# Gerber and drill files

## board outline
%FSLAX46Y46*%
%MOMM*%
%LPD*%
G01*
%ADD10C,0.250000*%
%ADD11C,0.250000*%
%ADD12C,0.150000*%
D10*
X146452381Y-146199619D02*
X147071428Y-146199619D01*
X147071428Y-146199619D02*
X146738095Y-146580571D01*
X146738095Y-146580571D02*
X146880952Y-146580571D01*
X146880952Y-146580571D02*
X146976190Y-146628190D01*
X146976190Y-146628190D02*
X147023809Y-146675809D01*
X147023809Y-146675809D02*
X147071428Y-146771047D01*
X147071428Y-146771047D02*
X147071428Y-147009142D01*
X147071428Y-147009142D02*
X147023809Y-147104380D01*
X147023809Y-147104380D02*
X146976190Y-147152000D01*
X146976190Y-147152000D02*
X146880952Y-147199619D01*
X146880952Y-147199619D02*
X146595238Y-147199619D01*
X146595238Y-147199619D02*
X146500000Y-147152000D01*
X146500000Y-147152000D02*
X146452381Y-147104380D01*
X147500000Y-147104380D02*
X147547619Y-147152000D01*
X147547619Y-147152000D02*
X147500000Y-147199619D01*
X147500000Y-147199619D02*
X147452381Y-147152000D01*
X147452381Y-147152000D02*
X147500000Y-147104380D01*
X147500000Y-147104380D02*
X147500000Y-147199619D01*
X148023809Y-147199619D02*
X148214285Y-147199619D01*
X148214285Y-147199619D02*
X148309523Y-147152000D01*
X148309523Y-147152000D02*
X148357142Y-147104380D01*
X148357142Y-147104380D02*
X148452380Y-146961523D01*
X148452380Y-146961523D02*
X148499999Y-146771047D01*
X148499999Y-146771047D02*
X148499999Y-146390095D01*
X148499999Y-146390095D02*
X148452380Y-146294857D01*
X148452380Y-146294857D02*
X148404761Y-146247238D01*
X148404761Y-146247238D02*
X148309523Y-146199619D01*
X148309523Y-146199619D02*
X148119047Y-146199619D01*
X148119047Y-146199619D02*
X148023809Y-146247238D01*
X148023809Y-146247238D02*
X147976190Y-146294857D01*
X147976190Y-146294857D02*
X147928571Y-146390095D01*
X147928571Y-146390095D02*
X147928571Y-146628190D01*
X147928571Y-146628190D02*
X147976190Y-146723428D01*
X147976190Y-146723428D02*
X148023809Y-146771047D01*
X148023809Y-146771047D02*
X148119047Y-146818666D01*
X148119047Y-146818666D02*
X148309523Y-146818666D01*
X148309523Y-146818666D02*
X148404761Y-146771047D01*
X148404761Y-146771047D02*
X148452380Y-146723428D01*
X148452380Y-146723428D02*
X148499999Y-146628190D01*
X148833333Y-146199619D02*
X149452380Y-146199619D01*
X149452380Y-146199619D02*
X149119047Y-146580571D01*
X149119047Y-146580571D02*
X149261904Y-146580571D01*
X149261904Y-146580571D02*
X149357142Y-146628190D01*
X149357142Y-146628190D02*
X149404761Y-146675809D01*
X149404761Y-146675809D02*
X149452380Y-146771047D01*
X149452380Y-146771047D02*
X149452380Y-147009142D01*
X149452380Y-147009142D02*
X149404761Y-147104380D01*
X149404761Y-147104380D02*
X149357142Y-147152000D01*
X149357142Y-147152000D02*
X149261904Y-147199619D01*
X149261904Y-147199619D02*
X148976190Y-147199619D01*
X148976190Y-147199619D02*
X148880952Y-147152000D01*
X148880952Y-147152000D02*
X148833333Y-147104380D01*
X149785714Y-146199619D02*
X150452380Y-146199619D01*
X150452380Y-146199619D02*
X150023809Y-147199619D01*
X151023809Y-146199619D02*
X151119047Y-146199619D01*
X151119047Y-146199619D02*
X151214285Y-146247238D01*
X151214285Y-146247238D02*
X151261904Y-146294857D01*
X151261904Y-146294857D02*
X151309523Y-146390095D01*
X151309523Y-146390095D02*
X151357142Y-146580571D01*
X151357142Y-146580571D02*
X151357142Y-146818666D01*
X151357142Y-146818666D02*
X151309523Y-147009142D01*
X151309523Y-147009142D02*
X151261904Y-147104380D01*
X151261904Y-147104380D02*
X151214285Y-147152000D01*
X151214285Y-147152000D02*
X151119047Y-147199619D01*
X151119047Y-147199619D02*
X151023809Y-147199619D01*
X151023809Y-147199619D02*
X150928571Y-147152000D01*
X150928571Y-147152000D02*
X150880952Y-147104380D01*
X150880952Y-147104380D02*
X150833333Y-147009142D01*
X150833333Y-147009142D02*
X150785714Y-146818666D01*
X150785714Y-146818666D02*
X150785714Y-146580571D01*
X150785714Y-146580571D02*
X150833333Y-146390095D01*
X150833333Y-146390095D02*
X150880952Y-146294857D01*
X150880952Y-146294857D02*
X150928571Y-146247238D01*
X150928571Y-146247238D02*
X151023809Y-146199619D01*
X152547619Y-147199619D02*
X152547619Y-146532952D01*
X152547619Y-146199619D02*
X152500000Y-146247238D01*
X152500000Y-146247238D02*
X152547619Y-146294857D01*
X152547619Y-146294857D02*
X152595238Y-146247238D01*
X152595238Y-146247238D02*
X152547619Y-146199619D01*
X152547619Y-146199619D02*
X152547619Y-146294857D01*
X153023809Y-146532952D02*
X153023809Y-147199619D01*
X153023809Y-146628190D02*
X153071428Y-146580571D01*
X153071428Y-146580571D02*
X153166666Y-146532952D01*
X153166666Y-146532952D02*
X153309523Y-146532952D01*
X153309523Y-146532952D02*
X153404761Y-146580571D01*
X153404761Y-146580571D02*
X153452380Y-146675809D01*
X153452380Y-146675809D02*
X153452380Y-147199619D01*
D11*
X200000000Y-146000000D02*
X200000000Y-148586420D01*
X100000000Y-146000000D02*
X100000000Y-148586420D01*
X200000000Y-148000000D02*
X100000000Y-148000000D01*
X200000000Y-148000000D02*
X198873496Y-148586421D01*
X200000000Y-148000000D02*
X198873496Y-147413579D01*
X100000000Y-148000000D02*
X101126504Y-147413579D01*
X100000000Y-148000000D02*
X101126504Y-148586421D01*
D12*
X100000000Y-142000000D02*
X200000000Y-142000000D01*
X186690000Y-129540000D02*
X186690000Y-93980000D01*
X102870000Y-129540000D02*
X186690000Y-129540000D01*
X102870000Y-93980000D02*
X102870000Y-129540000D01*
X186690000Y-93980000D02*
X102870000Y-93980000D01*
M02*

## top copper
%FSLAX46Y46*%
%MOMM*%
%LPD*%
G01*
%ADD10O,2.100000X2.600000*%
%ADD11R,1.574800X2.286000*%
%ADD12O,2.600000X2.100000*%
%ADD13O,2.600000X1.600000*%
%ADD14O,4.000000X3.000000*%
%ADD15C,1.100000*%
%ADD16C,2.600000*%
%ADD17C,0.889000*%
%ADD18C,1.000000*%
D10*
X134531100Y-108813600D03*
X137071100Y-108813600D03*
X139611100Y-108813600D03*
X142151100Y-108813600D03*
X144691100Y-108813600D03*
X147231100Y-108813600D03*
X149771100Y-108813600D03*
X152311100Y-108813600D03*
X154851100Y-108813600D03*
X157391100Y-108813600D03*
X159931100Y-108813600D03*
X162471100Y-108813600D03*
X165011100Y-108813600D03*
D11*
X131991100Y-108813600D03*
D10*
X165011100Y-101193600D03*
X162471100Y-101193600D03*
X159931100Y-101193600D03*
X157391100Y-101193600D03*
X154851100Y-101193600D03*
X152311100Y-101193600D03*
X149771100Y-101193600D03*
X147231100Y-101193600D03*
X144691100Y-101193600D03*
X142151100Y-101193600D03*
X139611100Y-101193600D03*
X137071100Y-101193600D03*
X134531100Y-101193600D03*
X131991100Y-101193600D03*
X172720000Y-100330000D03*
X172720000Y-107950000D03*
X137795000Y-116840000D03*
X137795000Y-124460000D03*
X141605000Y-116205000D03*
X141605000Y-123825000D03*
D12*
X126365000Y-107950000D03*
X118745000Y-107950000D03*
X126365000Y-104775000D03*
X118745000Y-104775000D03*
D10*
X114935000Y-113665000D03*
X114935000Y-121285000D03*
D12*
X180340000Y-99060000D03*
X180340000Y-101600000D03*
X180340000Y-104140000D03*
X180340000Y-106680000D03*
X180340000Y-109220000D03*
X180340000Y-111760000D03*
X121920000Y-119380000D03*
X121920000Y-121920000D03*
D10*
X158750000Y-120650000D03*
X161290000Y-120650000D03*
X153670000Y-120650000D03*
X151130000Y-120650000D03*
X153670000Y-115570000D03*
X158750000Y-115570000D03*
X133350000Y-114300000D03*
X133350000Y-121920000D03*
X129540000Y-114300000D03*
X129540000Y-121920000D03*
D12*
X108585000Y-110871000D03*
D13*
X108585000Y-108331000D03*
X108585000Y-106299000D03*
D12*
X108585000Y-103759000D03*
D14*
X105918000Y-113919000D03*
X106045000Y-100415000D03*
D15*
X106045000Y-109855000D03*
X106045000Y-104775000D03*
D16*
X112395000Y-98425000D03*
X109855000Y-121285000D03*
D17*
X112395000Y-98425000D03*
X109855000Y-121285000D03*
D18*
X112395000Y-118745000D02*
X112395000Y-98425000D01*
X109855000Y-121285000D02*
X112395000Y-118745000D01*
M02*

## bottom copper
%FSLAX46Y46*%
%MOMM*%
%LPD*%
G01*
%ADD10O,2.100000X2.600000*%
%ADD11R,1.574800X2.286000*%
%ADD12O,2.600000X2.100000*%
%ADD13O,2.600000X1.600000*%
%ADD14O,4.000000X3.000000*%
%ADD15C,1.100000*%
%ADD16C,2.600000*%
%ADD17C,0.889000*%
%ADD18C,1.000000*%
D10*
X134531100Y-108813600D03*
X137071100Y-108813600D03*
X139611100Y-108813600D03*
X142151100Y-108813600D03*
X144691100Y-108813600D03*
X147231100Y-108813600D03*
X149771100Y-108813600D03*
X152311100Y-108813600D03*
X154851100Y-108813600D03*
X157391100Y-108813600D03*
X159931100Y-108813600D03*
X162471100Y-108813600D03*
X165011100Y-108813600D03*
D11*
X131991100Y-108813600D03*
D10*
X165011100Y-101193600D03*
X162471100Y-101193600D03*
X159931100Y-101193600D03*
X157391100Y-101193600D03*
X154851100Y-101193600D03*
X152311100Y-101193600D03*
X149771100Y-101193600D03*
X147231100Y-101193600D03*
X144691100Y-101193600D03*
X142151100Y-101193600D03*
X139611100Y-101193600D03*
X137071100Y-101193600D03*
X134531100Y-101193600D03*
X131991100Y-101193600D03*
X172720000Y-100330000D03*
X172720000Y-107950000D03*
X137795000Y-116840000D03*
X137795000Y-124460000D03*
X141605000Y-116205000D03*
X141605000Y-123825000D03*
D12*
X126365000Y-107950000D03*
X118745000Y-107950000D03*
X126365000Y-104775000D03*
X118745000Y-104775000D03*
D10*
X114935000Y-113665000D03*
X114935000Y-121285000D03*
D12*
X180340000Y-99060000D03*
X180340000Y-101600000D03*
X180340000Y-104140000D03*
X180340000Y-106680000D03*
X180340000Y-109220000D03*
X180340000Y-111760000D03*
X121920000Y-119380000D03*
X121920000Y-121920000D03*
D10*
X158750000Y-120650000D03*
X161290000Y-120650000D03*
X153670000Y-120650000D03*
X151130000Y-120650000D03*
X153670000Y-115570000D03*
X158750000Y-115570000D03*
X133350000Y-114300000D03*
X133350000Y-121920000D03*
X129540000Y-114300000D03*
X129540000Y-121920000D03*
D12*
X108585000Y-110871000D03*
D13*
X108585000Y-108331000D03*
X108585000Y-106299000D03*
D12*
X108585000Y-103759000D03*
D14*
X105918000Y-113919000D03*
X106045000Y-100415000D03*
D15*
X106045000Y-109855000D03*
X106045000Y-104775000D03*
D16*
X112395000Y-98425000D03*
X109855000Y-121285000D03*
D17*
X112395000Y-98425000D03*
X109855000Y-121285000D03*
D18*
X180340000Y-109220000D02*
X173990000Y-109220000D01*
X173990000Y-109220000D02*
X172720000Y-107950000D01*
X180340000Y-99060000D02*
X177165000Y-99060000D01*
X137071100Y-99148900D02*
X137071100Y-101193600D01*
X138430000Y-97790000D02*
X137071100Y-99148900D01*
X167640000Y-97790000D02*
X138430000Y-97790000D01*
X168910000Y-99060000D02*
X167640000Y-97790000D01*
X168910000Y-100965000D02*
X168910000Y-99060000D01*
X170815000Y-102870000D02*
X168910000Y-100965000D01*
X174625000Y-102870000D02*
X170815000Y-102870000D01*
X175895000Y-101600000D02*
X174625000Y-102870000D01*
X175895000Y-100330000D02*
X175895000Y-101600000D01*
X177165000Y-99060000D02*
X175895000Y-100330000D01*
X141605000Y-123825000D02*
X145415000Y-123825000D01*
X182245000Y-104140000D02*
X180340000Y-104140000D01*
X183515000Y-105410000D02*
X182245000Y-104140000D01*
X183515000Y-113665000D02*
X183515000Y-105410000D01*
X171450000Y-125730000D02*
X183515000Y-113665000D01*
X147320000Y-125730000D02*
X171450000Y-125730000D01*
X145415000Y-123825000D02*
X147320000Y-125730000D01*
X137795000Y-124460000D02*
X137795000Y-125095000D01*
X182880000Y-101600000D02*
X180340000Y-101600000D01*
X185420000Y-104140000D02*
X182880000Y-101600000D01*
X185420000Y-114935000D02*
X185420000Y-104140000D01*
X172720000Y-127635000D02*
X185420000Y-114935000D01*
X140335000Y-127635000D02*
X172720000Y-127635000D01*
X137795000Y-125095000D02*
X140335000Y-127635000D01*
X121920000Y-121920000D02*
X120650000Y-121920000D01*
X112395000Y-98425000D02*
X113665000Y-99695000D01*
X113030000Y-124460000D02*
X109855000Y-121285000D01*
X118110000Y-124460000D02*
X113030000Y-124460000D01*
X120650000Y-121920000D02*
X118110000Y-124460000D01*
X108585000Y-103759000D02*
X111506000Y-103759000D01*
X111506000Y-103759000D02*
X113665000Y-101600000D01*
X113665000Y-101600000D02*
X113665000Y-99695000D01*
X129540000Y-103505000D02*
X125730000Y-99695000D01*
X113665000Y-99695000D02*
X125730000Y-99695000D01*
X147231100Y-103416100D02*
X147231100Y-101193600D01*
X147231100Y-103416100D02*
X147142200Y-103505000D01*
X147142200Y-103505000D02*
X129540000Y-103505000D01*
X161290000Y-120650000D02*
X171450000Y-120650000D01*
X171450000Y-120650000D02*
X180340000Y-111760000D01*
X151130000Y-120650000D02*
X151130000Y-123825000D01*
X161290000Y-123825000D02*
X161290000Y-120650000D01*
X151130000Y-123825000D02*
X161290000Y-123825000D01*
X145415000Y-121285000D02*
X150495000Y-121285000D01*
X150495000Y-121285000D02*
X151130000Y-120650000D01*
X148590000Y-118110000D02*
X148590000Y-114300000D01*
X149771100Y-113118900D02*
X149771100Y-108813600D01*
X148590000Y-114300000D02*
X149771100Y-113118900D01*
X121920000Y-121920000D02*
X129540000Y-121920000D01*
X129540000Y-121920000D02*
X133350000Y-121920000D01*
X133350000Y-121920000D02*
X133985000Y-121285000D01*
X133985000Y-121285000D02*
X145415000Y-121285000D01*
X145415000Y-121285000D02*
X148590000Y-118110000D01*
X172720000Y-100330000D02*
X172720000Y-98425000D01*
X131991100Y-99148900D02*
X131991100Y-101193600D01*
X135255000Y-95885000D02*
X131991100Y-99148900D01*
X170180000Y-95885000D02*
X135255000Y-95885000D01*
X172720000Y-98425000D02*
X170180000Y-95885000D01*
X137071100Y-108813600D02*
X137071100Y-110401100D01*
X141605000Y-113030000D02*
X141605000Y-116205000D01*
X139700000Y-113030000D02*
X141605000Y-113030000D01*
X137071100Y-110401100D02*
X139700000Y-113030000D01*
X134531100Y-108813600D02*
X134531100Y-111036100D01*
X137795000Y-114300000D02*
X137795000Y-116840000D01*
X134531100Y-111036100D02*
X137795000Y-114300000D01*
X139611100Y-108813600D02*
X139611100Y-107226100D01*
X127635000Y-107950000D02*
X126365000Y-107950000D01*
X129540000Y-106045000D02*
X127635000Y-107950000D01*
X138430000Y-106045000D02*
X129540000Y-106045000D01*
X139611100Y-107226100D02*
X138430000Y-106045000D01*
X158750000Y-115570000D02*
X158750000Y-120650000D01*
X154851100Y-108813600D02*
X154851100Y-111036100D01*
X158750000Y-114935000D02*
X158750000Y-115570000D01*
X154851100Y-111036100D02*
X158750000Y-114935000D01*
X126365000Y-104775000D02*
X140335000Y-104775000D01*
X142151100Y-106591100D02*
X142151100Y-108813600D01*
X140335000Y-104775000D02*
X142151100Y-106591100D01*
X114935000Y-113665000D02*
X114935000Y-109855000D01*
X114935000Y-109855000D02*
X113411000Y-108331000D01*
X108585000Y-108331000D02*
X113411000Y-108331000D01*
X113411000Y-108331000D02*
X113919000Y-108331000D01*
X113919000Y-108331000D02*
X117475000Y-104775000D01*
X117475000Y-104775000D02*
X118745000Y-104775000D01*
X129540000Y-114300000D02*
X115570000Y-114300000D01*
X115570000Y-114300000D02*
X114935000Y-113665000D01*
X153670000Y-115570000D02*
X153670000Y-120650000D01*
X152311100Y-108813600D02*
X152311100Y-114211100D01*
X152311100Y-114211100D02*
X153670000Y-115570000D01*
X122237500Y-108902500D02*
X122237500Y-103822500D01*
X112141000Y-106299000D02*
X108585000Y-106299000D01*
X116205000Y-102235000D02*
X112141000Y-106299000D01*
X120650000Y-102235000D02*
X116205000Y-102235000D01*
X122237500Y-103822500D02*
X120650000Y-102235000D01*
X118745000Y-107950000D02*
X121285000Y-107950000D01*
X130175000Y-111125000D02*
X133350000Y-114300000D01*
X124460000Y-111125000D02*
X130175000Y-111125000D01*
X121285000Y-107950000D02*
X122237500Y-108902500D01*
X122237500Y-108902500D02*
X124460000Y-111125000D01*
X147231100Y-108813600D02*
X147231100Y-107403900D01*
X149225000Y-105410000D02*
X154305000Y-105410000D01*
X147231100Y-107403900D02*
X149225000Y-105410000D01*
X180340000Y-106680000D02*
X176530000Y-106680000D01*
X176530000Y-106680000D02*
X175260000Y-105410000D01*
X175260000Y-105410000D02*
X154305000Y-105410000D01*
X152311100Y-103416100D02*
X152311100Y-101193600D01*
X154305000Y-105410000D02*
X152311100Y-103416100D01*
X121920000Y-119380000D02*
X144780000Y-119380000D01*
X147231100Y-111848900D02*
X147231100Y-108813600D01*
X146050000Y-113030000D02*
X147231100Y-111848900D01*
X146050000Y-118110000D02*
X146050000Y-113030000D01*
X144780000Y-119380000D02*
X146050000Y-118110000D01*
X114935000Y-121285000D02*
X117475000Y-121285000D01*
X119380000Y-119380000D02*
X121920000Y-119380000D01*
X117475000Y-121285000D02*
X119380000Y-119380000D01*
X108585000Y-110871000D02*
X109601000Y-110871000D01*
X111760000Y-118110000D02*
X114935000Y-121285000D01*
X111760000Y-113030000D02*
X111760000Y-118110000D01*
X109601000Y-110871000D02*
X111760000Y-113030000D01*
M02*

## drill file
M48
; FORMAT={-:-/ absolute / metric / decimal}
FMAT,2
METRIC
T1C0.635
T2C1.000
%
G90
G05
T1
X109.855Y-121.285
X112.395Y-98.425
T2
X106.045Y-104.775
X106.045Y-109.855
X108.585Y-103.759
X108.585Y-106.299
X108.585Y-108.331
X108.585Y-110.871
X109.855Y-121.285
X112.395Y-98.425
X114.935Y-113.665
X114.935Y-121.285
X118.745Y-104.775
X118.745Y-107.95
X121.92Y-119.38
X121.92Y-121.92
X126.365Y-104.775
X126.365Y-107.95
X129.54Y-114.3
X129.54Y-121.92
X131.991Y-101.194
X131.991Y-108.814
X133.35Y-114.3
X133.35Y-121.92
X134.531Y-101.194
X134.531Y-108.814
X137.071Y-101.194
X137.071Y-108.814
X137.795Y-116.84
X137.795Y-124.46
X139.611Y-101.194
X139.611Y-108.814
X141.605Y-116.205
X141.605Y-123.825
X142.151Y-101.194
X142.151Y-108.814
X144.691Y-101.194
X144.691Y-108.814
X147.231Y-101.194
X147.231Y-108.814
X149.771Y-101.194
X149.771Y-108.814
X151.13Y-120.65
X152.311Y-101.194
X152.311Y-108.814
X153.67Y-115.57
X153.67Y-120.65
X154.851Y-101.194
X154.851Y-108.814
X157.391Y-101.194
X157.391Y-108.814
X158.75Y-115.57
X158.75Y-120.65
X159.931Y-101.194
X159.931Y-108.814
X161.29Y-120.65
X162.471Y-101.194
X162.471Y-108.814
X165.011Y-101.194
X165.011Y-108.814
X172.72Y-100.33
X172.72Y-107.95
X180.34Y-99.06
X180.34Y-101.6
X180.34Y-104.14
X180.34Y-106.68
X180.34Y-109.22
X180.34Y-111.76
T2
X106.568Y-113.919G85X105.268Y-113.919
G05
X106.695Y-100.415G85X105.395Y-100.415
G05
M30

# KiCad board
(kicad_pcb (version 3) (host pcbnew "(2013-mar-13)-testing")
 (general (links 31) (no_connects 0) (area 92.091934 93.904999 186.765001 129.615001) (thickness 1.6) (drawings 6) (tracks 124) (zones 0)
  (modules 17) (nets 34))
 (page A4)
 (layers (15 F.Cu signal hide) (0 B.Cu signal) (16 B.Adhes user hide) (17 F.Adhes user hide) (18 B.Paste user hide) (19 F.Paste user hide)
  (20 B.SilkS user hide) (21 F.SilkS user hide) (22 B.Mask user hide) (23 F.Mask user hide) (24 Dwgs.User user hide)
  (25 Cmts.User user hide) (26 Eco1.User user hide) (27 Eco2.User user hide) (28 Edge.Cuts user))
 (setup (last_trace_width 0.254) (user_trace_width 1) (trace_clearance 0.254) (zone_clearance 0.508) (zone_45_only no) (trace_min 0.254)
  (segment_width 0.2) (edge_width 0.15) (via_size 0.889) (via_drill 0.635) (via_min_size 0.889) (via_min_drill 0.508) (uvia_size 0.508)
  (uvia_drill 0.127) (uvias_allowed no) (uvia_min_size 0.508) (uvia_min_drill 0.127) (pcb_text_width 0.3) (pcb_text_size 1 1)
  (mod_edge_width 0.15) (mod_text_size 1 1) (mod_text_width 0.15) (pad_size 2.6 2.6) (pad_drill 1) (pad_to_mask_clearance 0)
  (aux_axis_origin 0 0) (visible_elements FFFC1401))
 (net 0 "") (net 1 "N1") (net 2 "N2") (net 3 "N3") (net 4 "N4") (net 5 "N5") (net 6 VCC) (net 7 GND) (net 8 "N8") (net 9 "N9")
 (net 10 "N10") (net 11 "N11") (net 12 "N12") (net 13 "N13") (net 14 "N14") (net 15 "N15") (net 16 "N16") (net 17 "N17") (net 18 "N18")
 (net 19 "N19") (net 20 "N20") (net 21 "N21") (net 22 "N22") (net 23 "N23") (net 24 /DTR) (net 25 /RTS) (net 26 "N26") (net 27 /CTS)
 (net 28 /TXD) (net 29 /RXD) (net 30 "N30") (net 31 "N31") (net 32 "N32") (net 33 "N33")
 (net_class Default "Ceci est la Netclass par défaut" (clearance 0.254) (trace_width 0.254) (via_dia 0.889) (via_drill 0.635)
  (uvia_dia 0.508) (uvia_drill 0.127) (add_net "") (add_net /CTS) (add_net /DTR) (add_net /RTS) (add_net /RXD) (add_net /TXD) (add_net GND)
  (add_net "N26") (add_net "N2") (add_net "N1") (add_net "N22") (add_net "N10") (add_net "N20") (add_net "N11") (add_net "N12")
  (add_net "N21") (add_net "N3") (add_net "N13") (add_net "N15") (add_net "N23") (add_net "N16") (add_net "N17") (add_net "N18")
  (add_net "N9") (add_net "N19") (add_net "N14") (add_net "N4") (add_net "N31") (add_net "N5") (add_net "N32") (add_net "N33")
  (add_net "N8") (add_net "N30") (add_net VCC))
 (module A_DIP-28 (layer F.Cu) (at 148.5011 105.0036)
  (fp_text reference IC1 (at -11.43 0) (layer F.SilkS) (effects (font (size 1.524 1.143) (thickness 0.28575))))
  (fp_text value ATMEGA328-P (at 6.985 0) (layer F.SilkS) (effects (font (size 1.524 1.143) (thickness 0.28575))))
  (pad 2 thru_hole oval (at -13.97 3.81) (size 2.1 2.6) (drill 1) (layers *.Cu *.Mask F.SilkS) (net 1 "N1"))
  (pad 3 thru_hole oval (at -11.43 3.81) (size 2.1 2.6) (drill 1) (layers *.Cu *.Mask F.SilkS) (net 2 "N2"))
  (pad 4 thru_hole oval (at -8.89 3.81) (size 2.1 2.6) (drill 1) (layers *.Cu *.Mask F.SilkS) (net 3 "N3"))
  (pad 5 thru_hole oval (at -6.35 3.81) (size 2.1 2.6) (drill 1) (layers *.Cu *.Mask F.SilkS) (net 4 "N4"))
  (pad 6 thru_hole oval (at -3.81 3.81) (size 2.1 2.6) (drill 1) (layers *.Cu *.Mask F.SilkS) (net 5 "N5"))
  (pad 7 thru_hole oval (at -1.27 3.81) (size 2.1 2.6) (drill 1) (layers *.Cu *.Mask F.SilkS) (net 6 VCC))
  (pad 8 thru_hole oval (at 1.27 3.81) (size 2.1 2.6) (drill 1) (layers *.Cu *.Mask F.SilkS) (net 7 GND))
  (pad 9 thru_hole oval (at 3.81 3.81) (size 2.1 2.6) (drill 1) (layers *.Cu *.Mask F.SilkS) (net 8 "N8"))
  (pad 10 thru_hole oval (at 6.35 3.81) (size 2.1 2.6) (drill 1) (layers *.Cu *.Mask F.SilkS) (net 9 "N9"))
  (pad 11 thru_hole oval (at 8.89 3.81) (size 2.1 2.6) (drill 1) (layers *.Cu *.Mask F.SilkS) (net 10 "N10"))
  (pad 12 thru_hole oval (at 11.43 3.81) (size 2.1 2.6) (drill 1) (layers *.Cu *.Mask F.SilkS) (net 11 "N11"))
  (pad 13 thru_hole oval (at 13.97 3.81) (size 2.1 2.6) (drill 1) (layers *.Cu *.Mask F.SilkS) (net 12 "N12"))
  (pad 14 thru_hole oval (at 16.51 3.81) (size 2.1 2.6) (drill 1) (layers *.Cu *.Mask F.SilkS) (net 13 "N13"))
  (pad 1 thru_hole rect (at -16.51 3.81) (size 1.5748 2.286) (drill 1) (layers *.Cu *.Mask F.SilkS) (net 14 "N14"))
  (pad 15 thru_hole oval (at 16.51 -3.81) (size 2.1 2.6) (drill 1) (layers *.Cu *.Mask F.SilkS) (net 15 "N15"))
  (pad 16 thru_hole oval (at 13.97 -3.81) (size 2.1 2.6) (drill 1) (layers *.Cu *.Mask F.SilkS) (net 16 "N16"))
  (pad 17 thru_hole oval (at 11.43 -3.81) (size 2.1 2.6) (drill 1) (layers *.Cu *.Mask F.SilkS) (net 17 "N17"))
  (pad 18 thru_hole oval (at 8.89 -3.81) (size 2.1 2.6) (drill 1) (layers *.Cu *.Mask F.SilkS) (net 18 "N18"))
  (pad 19 thru_hole oval (at 6.35 -3.81) (size 2.1 2.6) (drill 1) (layers *.Cu *.Mask F.SilkS) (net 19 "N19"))
  (pad 20 thru_hole oval (at 3.81 -3.81) (size 2.1 2.6) (drill 1) (layers *.Cu *.Mask F.SilkS) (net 6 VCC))
  (pad 21 thru_hole oval (at 1.27 -3.81) (size 2.1 2.6) (drill 1) (layers *.Cu *.Mask F.SilkS) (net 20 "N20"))
  (pad 22 thru_hole oval (at -1.27 -3.81) (size 2.1 2.6) (drill 1) (layers *.Cu *.Mask F.SilkS) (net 7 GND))
  (pad 23 thru_hole oval (at -3.81 -3.81) (size 2.1 2.6) (drill 1) (layers *.Cu *.Mask F.SilkS) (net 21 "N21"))
  (pad 24 thru_hole oval (at -6.35 -3.81) (size 2.1 2.6) (drill 1) (layers *.Cu *.Mask F.SilkS) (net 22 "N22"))
  (pad 25 thru_hole oval (at -8.89 -3.81) (size 2.1 2.6) (drill 1) (layers *.Cu *.Mask F.SilkS) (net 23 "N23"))
  (pad 26 thru_hole oval (at -11.43 -3.81) (size 2.1 2.6) (drill 1) (layers *.Cu *.Mask F.SilkS) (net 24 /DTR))
  (pad 27 thru_hole oval (at -13.97 -3.81) (size 2.1 2.6) (drill 1) (layers *.Cu *.Mask F.SilkS) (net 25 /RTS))
  (pad 28 thru_hole oval (at -16.51 -3.81) (size 2.1 2.6) (drill 1) (layers *.Cu *.Mask F.SilkS) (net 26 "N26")))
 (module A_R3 (layer F.Cu) (at 172.72 104.14 270) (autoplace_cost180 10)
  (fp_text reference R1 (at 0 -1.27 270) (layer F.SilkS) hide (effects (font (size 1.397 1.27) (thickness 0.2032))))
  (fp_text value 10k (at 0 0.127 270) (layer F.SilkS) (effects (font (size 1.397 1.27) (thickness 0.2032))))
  (pad 1 thru_hole oval (at -3.81 0 270) (size 2.6 2.1) (drill 1) (layers *.Cu *.Mask F.SilkS) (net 26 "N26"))
  (pad 2 thru_hole oval (at 3.81 0 270) (size 2.6 2.1) (drill 1) (layers *.Cu *.Mask F.SilkS) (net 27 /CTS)))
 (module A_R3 (layer F.Cu) (at 137.795 120.65 270) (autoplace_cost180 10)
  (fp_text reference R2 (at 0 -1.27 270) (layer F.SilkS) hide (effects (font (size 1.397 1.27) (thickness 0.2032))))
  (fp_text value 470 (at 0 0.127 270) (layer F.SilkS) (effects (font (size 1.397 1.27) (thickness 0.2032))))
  (pad 1 thru_hole oval (at -3.81 0 270) (size 2.6 2.1) (drill 1) (layers *.Cu *.Mask F.SilkS) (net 1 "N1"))
  (pad 2 thru_hole oval (at 3.81 0 270) (size 2.6 2.1) (drill 1) (layers *.Cu *.Mask F.SilkS) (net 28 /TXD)))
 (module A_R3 (layer F.Cu) (at 141.605 120.015 270) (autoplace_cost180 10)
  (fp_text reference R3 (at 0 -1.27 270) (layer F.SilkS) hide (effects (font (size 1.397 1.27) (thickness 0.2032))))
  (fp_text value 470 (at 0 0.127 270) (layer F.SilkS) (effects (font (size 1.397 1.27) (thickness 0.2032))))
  (pad 1 thru_hole oval (at -3.81 0 270) (size 2.6 2.1) (drill 1) (layers *.Cu *.Mask F.SilkS) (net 2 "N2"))
  (pad 2 thru_hole oval (at 3.81 0 270) (size 2.6 2.1) (drill 1) (layers *.Cu *.Mask F.SilkS) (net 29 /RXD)))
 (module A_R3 (layer F.Cu) (at 122.555 107.95 180) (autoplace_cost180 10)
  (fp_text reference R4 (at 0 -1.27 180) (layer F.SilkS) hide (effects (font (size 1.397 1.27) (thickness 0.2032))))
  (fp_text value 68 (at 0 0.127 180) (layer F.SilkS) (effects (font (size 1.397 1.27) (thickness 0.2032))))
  (pad 1 thru_hole oval (at -3.81 0 180) (size 2.6 2.1) (drill 1) (layers *.Cu *.Mask F.SilkS) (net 3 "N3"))
  (pad 2 thru_hole oval (at 3.81 0 180) (size 2.6 2.1) (drill 1) (layers *.Cu *.Mask F.SilkS) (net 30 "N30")))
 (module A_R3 (layer F.Cu) (at 122.555 104.775 180) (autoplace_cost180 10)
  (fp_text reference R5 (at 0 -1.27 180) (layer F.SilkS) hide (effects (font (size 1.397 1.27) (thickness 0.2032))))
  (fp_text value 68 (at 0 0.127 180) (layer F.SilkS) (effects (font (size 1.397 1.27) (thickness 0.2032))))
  (pad 1 thru_hole oval (at -3.81 0 180) (size 2.6 2.1) (drill 1) (layers *.Cu *.Mask F.SilkS) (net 4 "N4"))
  (pad 2 thru_hole oval (at 3.81 0 180) (size 2.6 2.1) (drill 1) (layers *.Cu *.Mask F.SilkS) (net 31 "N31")))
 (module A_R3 (layer F.Cu) (at 114.935 117.475 270) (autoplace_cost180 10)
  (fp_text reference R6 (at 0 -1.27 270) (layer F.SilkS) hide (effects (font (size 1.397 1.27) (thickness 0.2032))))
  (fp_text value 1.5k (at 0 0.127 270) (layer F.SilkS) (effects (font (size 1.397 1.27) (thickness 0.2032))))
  (pad 1 thru_hole oval (at -3.81 0 270) (size 2.6 2.1) (drill 1) (layers *.Cu *.Mask F.SilkS) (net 31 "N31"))
  (pad 2 thru_hole oval (at 3.81 0 270) (size 2.6 2.1) (drill 1) (layers *.Cu *.Mask F.SilkS) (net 6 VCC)))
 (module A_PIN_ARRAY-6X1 (layer F.Cu) (at 180.34 105.41 270)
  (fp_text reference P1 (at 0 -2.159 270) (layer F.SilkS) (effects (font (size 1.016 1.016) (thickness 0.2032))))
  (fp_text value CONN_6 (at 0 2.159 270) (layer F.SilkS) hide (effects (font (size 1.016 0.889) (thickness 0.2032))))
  (pad 1 thru_hole oval (at -6.35 0 270) (size 2.1 2.6) (drill 1) (layers *.Cu *.Mask F.SilkS) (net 24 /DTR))
  (pad 2 thru_hole oval (at -3.81 0 270) (size 2.1 2.6) (drill 1) (layers *.Cu *.Mask F.SilkS) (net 28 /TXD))
  (pad 3 thru_hole oval (at -1.27 0 270) (size 2.1 2.6) (drill 1) (layers *.Cu *.Mask F.SilkS) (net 29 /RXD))
  (pad 4 thru_hole oval (at 1.27 0 270) (size 2.1 2.6) (drill 1) (layers *.Cu *.Mask F.SilkS) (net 6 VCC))
  (pad 5 thru_hole oval (at 3.81 0 270) (size 2.1 2.6) (drill 1) (layers *.Cu *.Mask F.SilkS) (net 27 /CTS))
  (pad 6 thru_hole oval (at 6.35 0 270) (size 2.1 2.6) (drill 1) (layers *.Cu *.Mask F.SilkS) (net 7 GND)))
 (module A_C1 (layer F.Cu) (at 121.92 120.65 270)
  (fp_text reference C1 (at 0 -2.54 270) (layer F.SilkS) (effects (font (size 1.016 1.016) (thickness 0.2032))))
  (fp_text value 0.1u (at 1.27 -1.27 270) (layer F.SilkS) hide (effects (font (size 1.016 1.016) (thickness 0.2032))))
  (pad 1 thru_hole oval (at -1.27 0 270) (size 2.1 2.6) (drill 1) (layers *.Cu *.Mask F.SilkS) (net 6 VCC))
  (pad 2 thru_hole oval (at 1.27 0 270) (size 2.1 2.6) (drill 1) (layers *.Cu *.Mask F.SilkS) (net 7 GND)))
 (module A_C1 (layer F.Cu) (at 160.02 120.65)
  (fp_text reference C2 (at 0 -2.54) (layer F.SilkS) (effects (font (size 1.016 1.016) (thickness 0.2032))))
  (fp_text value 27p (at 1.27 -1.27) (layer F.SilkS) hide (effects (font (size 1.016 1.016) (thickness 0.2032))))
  (pad 1 thru_hole oval (at -1.27 0) (size 2.1 2.6) (drill 1) (layers *.Cu *.Mask F.SilkS) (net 9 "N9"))
  (pad 2 thru_hole oval (at 1.27 0) (size 2.1 2.6) (drill 1) (layers *.Cu *.Mask F.SilkS) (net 7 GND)))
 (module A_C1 (layer F.Cu) (at 152.4 120.65 180)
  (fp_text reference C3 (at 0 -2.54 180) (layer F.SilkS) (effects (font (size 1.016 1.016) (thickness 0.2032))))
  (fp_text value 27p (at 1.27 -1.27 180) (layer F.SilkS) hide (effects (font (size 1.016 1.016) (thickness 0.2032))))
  (pad 1 thru_hole oval (at -1.27 0 180) (size 2.1 2.6) (drill 1) (layers *.Cu *.Mask F.SilkS) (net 8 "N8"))
  (pad 2 thru_hole oval (at 1.27 0 180) (size 2.1 2.6) (drill 1) (layers *.Cu *.Mask F.SilkS) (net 7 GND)))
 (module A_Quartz (layer F.Cu) (at 154.94 115.57)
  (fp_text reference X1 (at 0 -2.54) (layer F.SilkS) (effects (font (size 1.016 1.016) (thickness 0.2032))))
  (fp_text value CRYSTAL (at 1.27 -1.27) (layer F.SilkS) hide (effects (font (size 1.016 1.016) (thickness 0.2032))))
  (pad 1 thru_hole oval (at -1.27 0) (size 2.1 2.6) (drill 1) (layers *.Cu *.Mask F.SilkS) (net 8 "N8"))
  (pad 2 thru_hole oval (at 3.81 0) (size 2.1 2.6) (drill 1) (layers *.Cu *.Mask F.SilkS) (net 9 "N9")))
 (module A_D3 (layer F.Cu) (at 133.35 118.11 90)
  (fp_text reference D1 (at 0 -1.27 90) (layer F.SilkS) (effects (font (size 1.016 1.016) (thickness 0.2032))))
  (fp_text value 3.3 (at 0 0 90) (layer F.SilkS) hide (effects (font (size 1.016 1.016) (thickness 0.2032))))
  (pad 2 thru_hole oval (at 3.81 0 90) (size 2.6 2.1) (drill 1) (layers *.Cu *.Mask F.SilkS) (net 30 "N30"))
  (pad 1 thru_hole oval (at -3.81 0 90) (size 2.6 2.1) (drill 1) (layers *.Cu *.Mask F.SilkS) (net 7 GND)))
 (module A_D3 (layer F.Cu) (at 129.54 118.11 90)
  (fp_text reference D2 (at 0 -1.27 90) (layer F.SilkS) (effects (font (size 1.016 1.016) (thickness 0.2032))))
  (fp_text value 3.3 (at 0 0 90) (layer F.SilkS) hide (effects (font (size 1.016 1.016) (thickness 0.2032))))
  (pad 2 thru_hole oval (at 3.81 0 90) (size 2.6 2.1) (drill 1) (layers *.Cu *.Mask F.SilkS) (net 31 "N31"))
  (pad 1 thru_hole oval (at -3.81 0 90) (size 2.6 2.1) (drill 1) (layers *.Cu *.Mask F.SilkS) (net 7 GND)))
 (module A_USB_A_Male (layer F.Cu) (at 108.585 107.315 180)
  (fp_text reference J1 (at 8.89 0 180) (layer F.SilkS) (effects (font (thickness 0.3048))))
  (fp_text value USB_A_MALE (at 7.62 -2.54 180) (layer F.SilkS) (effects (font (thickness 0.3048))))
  (pad 1 thru_hole oval (at 0 -3.556 180) (size 2.6 2.1) (drill 1) (layers *.Cu *.Mask F.SilkS) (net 6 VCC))
  (pad 2 thru_hole oval (at 0 -1.016 180) (size 2.6 1.6) (drill 1) (layers *.Cu *.Mask F.SilkS) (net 31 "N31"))
  (pad 3 thru_hole oval (at 0 1.016 180) (size 2.6 1.6) (drill 1) (layers *.Cu *.Mask F.SilkS) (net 30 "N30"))
  (pad 4 thru_hole oval (at 0 3.556 180) (size 2.6 2.1) (drill 1) (layers *.Cu *.Mask F.SilkS) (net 7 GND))
  (pad 6 thru_hole oval (at 2.667 -6.604 180) (size 4 3) (drill oval 2.3 1) (layers *.Cu *.Mask F.SilkS) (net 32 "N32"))
  (pad 5 thru_hole oval (at 2.54 6.9 180) (size 4 3) (drill oval 2.3 1) (layers *.Cu *.Mask F.SilkS) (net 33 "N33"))
  (pad "" thru_hole circle (at 2.54 -2.54 180) (size 1.1 1.1) (drill 1) (layers *.Cu *.Mask F.SilkS))
  (pad "" thru_hole circle (at 2.54 2.54 180) (size 1.1 1.1) (drill 1) (layers *.Cu *.Mask F.SilkS)))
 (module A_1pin (layer F.Cu) (at 112.395 98.425)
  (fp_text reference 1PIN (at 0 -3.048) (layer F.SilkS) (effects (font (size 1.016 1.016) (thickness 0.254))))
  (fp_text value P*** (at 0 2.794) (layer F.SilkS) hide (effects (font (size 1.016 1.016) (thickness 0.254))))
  (pad 1 thru_hole circle (at 0 0) (size 2.6 2.6) (drill 1) (layers *.Cu *.Mask F.SilkS)))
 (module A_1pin (layer F.Cu) (at 109.855 121.285)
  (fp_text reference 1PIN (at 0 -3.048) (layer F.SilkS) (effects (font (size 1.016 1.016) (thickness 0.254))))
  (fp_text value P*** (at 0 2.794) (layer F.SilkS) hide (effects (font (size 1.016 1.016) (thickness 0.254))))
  (pad 1 thru_hole circle (at 0 0) (size 2.6 2.6) (drill 1) (layers *.Cu *.Mask F.SilkS)))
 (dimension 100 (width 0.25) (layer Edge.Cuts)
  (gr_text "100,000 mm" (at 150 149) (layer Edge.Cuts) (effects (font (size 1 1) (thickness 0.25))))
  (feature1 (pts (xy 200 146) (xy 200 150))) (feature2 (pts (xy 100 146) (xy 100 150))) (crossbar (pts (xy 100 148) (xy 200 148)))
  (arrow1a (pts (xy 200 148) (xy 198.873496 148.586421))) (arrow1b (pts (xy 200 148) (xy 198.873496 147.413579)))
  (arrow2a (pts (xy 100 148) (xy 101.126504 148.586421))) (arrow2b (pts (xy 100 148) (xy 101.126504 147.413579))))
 (gr_line (start 100 142) (end 200 142) (angle 90) (layer Edge.Cuts) (width 0.15))
 (gr_line (start 186.69 129.54) (end 186.69 93.98) (angle 90) (layer Edge.Cuts) (width 0.15))
 (gr_line (start 102.87 129.54) (end 186.69 129.54) (angle 90) (layer Edge.Cuts) (width 0.15))
 (gr_line (start 102.87 93.98) (end 102.87 129.54) (angle 90) (layer Edge.Cuts) (width 0.15))
 (gr_line (start 186.69 93.98) (end 102.87 93.98) (angle 90) (layer Edge.Cuts) (width 0.15))
 (segment (start 180.34 109.22) (end 173.99 109.22) (width 1) (layer B.Cu) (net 27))
 (segment (start 173.99 109.22) (end 172.72 107.95) (width 1) (layer B.Cu) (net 27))
 (segment (start 180.34 99.06) (end 177.165 99.06) (width 1) (layer B.Cu) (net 24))
 (segment (start 137.0711 99.1489) (end 137.0711 101.1936) (width 1) (layer B.Cu) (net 24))
 (segment (start 138.43 97.79) (end 137.0711 99.1489) (width 1) (layer B.Cu) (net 24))
 (segment (start 167.64 97.79) (end 138.43 97.79) (width 1) (layer B.Cu) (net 24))
 (segment (start 168.91 99.06) (end 167.64 97.79) (width 1) (layer B.Cu) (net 24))
 (segment (start 168.91 100.965) (end 168.91 99.06) (width 1) (layer B.Cu) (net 24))
 (segment (start 170.815 102.87) (end 168.91 100.965) (width 1) (layer B.Cu) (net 24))
 (segment (start 174.625 102.87) (end 170.815 102.87) (width 1) (layer B.Cu) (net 24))
 (segment (start 175.895 101.6) (end 174.625 102.87) (width 1) (layer B.Cu) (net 24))
 (segment (start 175.895 100.33) (end 175.895 101.6) (width 1) (layer B.Cu) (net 24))
 (segment (start 177.165 99.06) (end 175.895 100.33) (width 1) (layer B.Cu) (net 24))
 (segment (start 141.605 123.825) (end 145.415 123.825) (width 1) (layer B.Cu) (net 29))
 (segment (start 182.245 104.14) (end 180.34 104.14) (width 1) (layer B.Cu) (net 29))
 (segment (start 183.515 105.41) (end 182.245 104.14) (width 1) (layer B.Cu) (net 29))
 (segment (start 183.515 113.665) (end 183.515 105.41) (width 1) (layer B.Cu) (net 29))
 (segment (start 171.45 125.73) (end 183.515 113.665) (width 1) (layer B.Cu) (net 29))
 (segment (start 147.32 125.73) (end 171.45 125.73) (width 1) (layer B.Cu) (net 29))
 (segment (start 145.415 123.825) (end 147.32 125.73) (width 1) (layer B.Cu) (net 29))
 (segment (start 137.795 124.46) (end 137.795 125.095) (width 1) (layer B.Cu) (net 28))
 (segment (start 182.88 101.6) (end 180.34 101.6) (width 1) (layer B.Cu) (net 28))
 (segment (start 185.42 104.14) (end 182.88 101.6) (width 1) (layer B.Cu) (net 28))
 (segment (start 185.42 114.935) (end 185.42 104.14) (width 1) (layer B.Cu) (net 28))
 (segment (start 172.72 127.635) (end 185.42 114.935) (width 1) (layer B.Cu) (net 28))
 (segment (start 140.335 127.635) (end 172.72 127.635) (width 1) (layer B.Cu) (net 28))
 (segment (start 137.795 125.095) (end 140.335 127.635) (width 1) (layer B.Cu) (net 28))
 (segment (start 121.92 121.92) (end 120.65 121.92) (width 1) (layer B.Cu) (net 7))
 (segment (start 112.395 98.425) (end 113.665 99.695) (width 1) (layer B.Cu) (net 7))
 (via (at 112.395 98.425) (size 0.889) (layers F.Cu B.Cu) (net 7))
 (segment (start 112.395 118.745) (end 112.395 98.425) (width 1) (layer F.Cu) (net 7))
 (segment (start 109.855 121.285) (end 112.395 118.745) (width 1) (layer F.Cu) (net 7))
 (via (at 109.855 121.285) (size 0.889) (layers F.Cu B.Cu) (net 7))
 (segment (start 113.03 124.46) (end 109.855 121.285) (width 1) (layer B.Cu) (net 7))
 (segment (start 118.11 124.46) (end 113.03 124.46) (width 1) (layer B.Cu) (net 7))
 (segment (start 120.65 121.92) (end 118.11 124.46) (width 1) (layer B.Cu) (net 7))
 (segment (start 108.585 103.759) (end 111.506 103.759) (width 1) (layer B.Cu) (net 7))
 (segment (start 111.506 103.759) (end 113.665 101.6) (width 1) (layer B.Cu) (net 7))
 (segment (start 113.665 101.6) (end 113.665 99.695) (width 1) (layer B.Cu) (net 7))
 (segment (start 129.54 103.505) (end 125.73 99.695) (width 1) (layer B.Cu) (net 7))
 (segment (start 113.665 99.695) (end 125.73 99.695) (width 1) (layer B.Cu) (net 7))
 (segment (start 147.2311 103.4161) (end 147.2311 101.1936) (width 1) (layer B.Cu) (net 7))
 (segment (start 147.2311 103.4161) (end 147.1422 103.505) (width 1) (layer B.Cu) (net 7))
 (segment (start 147.1422 103.505) (end 129.54 103.505) (width 1) (layer B.Cu) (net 7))
 (segment (start 161.29 120.65) (end 171.45 120.65) (width 1) (layer B.Cu) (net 7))
 (segment (start 171.45 120.65) (end 180.34 111.76) (width 1) (layer B.Cu) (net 7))
 (segment (start 151.13 120.65) (end 151.13 123.825) (width 1) (layer B.Cu) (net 7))
 (segment (start 161.29 123.825) (end 161.29 120.65) (width 1) (layer B.Cu) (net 7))
 (segment (start 151.13 123.825) (end 161.29 123.825) (width 1) (layer B.Cu) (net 7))
 (segment (start 145.415 121.285) (end 150.495 121.285) (width 1) (layer B.Cu) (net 7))
 (segment (start 150.495 121.285) (end 151.13 120.65) (width 1) (layer B.Cu) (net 7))
 (segment (start 148.59 118.11) (end 148.59 114.3) (width 1) (layer B.Cu) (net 7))
 (segment (start 149.7711 113.1189) (end 149.7711 108.8136) (width 1) (layer B.Cu) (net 7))
 (segment (start 148.59 114.3) (end 149.7711 113.1189) (width 1) (layer B.Cu) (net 7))
 (segment (start 121.92 121.92) (end 129.54 121.92) (width 1) (layer B.Cu) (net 7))
 (segment (start 129.54 121.92) (end 133.35 121.92) (width 1) (layer B.Cu) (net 7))
 (segment (start 133.35 121.92) (end 133.985 121.285) (width 1) (layer B.Cu) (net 7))
 (segment (start 133.985 121.285) (end 145.415 121.285) (width 1) (layer B.Cu) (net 7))
 (segment (start 145.415 121.285) (end 148.59 118.11) (width 1) (layer B.Cu) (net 7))
 (segment (start 172.72 100.33) (end 172.72 98.425) (width 1) (layer B.Cu) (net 26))
 (segment (start 131.9911 99.1489) (end 131.9911 101.1936) (width 1) (layer B.Cu) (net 26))
 (segment (start 135.255 95.885) (end 131.9911 99.1489) (width 1) (layer B.Cu) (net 26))
 (segment (start 170.18 95.885) (end 135.255 95.885) (width 1) (layer B.Cu) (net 26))
 (segment (start 172.72 98.425) (end 170.18 95.885) (width 1) (layer B.Cu) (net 26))
 (segment (start 137.0711 108.8136) (end 137.0711 110.4011) (width 1) (layer B.Cu) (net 2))
 (segment (start 141.605 113.03) (end 141.605 116.205) (width 1) (layer B.Cu) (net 2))
 (segment (start 139.7 113.03) (end 141.605 113.03) (width 1) (layer B.Cu) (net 2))
 (segment (start 137.0711 110.4011) (end 139.7 113.03) (width 1) (layer B.Cu) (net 2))
 (segment (start 134.5311 108.8136) (end 134.5311 111.0361) (width 1) (layer B.Cu) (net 1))
 (segment (start 137.795 114.3) (end 137.795 116.84) (width 1) (layer B.Cu) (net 1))
 (segment (start 134.5311 111.0361) (end 137.795 114.3) (width 1) (layer B.Cu) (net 1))
 (segment (start 139.6111 108.8136) (end 139.6111 107.2261) (width 1) (layer B.Cu) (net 3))
 (segment (start 127.635 107.95) (end 126.365 107.95) (width 1) (layer B.Cu) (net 3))
 (segment (start 129.54 106.045) (end 127.635 107.95) (width 1) (layer B.Cu) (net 3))
 (segment (start 138.43 106.045) (end 129.54 106.045) (width 1) (layer B.Cu) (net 3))
 (segment (start 139.6111 107.2261) (end 138.43 106.045) (width 1) (layer B.Cu) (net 3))
 (segment (start 158.75 115.57) (end 158.75 120.65) (width 1) (layer B.Cu) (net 9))
 (segment (start 154.8511 108.8136) (end 154.8511 111.0361) (width 1) (layer B.Cu) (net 9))
 (segment (start 158.75 114.935) (end 158.75 115.57) (width 1) (layer B.Cu) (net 9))
 (segment (start 154.8511 111.0361) (end 158.75 114.935) (width 1) (layer B.Cu) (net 9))
 (segment (start 126.365 104.775) (end 140.335 104.775) (width 1) (layer B.Cu) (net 4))
 (segment (start 142.1511 106.5911) (end 142.1511 108.8136) (width 1) (layer B.Cu) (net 4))
 (segment (start 140.335 104.775) (end 142.1511 106.5911) (width 1) (layer B.Cu) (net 4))
 (segment (start 114.935 113.665) (end 114.935 109.855) (width 1) (layer B.Cu) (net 31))
 (segment (start 114.935 109.855) (end 113.411 108.331) (width 1) (layer B.Cu) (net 31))
 (segment (start 108.585 108.331) (end 113.411 108.331) (width 1) (layer B.Cu) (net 31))
 (segment (start 113.411 108.331) (end 113.919 108.331) (width 1) (layer B.Cu) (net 31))
 (segment (start 113.919 108.331) (end 117.475 104.775) (width 1) (layer B.Cu) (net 31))
 (segment (start 117.475 104.775) (end 118.745 104.775) (width 1) (layer B.Cu) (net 31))
 (segment (start 129.54 114.3) (end 115.57 114.3) (width 1) (layer B.Cu) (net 31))
 (segment (start 115.57 114.3) (end 114.935 113.665) (width 1) (layer B.Cu) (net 31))
 (segment (start 153.67 115.57) (end 153.67 120.65) (width 1) (layer B.Cu) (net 8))
 (segment (start 152.3111 108.8136) (end 152.3111 114.2111) (width 1) (layer B.Cu) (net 8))
 (segment (start 152.3111 114.2111) (end 153.67 115.57) (width 1) (layer B.Cu) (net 8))
 (segment (start 122.2375 108.9025) (end 122.2375 103.8225) (width 1) (layer B.Cu) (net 30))
 (segment (start 112.141 106.299) (end 108.585 106.299) (width 1) (layer B.Cu) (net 30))
 (segment (start 116.205 102.235) (end 112.141 106.299) (width 1) (layer B.Cu) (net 30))
 (segment (start 120.65 102.235) (end 116.205 102.235) (width 1) (layer B.Cu) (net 30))
 (segment (start 122.2375 103.8225) (end 120.65 102.235) (width 1) (layer B.Cu) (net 30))
 (segment (start 118.745 107.95) (end 121.285 107.95) (width 1) (layer B.Cu) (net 30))
 (segment (start 130.175 111.125) (end 133.35 114.3) (width 1) (layer B.Cu) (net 30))
 (segment (start 124.46 111.125) (end 130.175 111.125) (width 1) (layer B.Cu) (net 30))
 (segment (start 121.285 107.95) (end 122.2375 108.9025) (width 1) (layer B.Cu) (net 30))
 (segment (start 122.2375 108.9025) (end 124.46 111.125) (width 1) (layer B.Cu) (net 30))
 (segment (start 147.2311 108.8136) (end 147.2311 107.4039) (width 1) (layer B.Cu) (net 6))
 (segment (start 149.225 105.41) (end 154.305 105.41) (width 1) (layer B.Cu) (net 6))
 (segment (start 147.2311 107.4039) (end 149.225 105.41) (width 1) (layer B.Cu) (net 6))
 (segment (start 180.34 106.68) (end 176.53 106.68) (width 1) (layer B.Cu) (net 6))
 (segment (start 176.53 106.68) (end 175.26 105.41) (width 1) (layer B.Cu) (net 6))
 (segment (start 175.26 105.41) (end 154.305 105.41) (width 1) (layer B.Cu) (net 6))
 (segment (start 152.3111 103.4161) (end 152.3111 101.1936) (width 1) (layer B.Cu) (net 6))
 (segment (start 154.305 105.41) (end 152.3111 103.4161) (width 1) (layer B.Cu) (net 6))
 (segment (start 121.92 119.38) (end 144.78 119.38) (width 1) (layer B.Cu) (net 6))
 (segment (start 147.2311 111.8489) (end 147.2311 108.8136) (width 1) (layer B.Cu) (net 6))
 (segment (start 146.05 113.03) (end 147.2311 111.8489) (width 1) (layer B.Cu) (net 6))
 (segment (start 146.05 118.11) (end 146.05 113.03) (width 1) (layer B.Cu) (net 6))
 (segment (start 144.78 119.38) (end 146.05 118.11) (width 1) (layer B.Cu) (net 6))
 (segment (start 114.935 121.285) (end 117.475 121.285) (width 1) (layer B.Cu) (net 6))
 (segment (start 119.38 119.38) (end 121.92 119.38) (width 1) (layer B.Cu) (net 6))
 (segment (start 117.475 121.285) (end 119.38 119.38) (width 1) (layer B.Cu) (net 6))
 (segment (start 108.585 110.871) (end 109.601 110.871) (width 1) (layer B.Cu) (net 6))
 (segment (start 111.76 118.11) (end 114.935 121.285) (width 1) (layer B.Cu) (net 6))
 (segment (start 111.76 113.03) (end 111.76 118.11) (width 1) (layer B.Cu) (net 6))
 (segment (start 109.601 110.871) (end 111.76 113.03) (width 1) (layer B.Cu) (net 6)))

